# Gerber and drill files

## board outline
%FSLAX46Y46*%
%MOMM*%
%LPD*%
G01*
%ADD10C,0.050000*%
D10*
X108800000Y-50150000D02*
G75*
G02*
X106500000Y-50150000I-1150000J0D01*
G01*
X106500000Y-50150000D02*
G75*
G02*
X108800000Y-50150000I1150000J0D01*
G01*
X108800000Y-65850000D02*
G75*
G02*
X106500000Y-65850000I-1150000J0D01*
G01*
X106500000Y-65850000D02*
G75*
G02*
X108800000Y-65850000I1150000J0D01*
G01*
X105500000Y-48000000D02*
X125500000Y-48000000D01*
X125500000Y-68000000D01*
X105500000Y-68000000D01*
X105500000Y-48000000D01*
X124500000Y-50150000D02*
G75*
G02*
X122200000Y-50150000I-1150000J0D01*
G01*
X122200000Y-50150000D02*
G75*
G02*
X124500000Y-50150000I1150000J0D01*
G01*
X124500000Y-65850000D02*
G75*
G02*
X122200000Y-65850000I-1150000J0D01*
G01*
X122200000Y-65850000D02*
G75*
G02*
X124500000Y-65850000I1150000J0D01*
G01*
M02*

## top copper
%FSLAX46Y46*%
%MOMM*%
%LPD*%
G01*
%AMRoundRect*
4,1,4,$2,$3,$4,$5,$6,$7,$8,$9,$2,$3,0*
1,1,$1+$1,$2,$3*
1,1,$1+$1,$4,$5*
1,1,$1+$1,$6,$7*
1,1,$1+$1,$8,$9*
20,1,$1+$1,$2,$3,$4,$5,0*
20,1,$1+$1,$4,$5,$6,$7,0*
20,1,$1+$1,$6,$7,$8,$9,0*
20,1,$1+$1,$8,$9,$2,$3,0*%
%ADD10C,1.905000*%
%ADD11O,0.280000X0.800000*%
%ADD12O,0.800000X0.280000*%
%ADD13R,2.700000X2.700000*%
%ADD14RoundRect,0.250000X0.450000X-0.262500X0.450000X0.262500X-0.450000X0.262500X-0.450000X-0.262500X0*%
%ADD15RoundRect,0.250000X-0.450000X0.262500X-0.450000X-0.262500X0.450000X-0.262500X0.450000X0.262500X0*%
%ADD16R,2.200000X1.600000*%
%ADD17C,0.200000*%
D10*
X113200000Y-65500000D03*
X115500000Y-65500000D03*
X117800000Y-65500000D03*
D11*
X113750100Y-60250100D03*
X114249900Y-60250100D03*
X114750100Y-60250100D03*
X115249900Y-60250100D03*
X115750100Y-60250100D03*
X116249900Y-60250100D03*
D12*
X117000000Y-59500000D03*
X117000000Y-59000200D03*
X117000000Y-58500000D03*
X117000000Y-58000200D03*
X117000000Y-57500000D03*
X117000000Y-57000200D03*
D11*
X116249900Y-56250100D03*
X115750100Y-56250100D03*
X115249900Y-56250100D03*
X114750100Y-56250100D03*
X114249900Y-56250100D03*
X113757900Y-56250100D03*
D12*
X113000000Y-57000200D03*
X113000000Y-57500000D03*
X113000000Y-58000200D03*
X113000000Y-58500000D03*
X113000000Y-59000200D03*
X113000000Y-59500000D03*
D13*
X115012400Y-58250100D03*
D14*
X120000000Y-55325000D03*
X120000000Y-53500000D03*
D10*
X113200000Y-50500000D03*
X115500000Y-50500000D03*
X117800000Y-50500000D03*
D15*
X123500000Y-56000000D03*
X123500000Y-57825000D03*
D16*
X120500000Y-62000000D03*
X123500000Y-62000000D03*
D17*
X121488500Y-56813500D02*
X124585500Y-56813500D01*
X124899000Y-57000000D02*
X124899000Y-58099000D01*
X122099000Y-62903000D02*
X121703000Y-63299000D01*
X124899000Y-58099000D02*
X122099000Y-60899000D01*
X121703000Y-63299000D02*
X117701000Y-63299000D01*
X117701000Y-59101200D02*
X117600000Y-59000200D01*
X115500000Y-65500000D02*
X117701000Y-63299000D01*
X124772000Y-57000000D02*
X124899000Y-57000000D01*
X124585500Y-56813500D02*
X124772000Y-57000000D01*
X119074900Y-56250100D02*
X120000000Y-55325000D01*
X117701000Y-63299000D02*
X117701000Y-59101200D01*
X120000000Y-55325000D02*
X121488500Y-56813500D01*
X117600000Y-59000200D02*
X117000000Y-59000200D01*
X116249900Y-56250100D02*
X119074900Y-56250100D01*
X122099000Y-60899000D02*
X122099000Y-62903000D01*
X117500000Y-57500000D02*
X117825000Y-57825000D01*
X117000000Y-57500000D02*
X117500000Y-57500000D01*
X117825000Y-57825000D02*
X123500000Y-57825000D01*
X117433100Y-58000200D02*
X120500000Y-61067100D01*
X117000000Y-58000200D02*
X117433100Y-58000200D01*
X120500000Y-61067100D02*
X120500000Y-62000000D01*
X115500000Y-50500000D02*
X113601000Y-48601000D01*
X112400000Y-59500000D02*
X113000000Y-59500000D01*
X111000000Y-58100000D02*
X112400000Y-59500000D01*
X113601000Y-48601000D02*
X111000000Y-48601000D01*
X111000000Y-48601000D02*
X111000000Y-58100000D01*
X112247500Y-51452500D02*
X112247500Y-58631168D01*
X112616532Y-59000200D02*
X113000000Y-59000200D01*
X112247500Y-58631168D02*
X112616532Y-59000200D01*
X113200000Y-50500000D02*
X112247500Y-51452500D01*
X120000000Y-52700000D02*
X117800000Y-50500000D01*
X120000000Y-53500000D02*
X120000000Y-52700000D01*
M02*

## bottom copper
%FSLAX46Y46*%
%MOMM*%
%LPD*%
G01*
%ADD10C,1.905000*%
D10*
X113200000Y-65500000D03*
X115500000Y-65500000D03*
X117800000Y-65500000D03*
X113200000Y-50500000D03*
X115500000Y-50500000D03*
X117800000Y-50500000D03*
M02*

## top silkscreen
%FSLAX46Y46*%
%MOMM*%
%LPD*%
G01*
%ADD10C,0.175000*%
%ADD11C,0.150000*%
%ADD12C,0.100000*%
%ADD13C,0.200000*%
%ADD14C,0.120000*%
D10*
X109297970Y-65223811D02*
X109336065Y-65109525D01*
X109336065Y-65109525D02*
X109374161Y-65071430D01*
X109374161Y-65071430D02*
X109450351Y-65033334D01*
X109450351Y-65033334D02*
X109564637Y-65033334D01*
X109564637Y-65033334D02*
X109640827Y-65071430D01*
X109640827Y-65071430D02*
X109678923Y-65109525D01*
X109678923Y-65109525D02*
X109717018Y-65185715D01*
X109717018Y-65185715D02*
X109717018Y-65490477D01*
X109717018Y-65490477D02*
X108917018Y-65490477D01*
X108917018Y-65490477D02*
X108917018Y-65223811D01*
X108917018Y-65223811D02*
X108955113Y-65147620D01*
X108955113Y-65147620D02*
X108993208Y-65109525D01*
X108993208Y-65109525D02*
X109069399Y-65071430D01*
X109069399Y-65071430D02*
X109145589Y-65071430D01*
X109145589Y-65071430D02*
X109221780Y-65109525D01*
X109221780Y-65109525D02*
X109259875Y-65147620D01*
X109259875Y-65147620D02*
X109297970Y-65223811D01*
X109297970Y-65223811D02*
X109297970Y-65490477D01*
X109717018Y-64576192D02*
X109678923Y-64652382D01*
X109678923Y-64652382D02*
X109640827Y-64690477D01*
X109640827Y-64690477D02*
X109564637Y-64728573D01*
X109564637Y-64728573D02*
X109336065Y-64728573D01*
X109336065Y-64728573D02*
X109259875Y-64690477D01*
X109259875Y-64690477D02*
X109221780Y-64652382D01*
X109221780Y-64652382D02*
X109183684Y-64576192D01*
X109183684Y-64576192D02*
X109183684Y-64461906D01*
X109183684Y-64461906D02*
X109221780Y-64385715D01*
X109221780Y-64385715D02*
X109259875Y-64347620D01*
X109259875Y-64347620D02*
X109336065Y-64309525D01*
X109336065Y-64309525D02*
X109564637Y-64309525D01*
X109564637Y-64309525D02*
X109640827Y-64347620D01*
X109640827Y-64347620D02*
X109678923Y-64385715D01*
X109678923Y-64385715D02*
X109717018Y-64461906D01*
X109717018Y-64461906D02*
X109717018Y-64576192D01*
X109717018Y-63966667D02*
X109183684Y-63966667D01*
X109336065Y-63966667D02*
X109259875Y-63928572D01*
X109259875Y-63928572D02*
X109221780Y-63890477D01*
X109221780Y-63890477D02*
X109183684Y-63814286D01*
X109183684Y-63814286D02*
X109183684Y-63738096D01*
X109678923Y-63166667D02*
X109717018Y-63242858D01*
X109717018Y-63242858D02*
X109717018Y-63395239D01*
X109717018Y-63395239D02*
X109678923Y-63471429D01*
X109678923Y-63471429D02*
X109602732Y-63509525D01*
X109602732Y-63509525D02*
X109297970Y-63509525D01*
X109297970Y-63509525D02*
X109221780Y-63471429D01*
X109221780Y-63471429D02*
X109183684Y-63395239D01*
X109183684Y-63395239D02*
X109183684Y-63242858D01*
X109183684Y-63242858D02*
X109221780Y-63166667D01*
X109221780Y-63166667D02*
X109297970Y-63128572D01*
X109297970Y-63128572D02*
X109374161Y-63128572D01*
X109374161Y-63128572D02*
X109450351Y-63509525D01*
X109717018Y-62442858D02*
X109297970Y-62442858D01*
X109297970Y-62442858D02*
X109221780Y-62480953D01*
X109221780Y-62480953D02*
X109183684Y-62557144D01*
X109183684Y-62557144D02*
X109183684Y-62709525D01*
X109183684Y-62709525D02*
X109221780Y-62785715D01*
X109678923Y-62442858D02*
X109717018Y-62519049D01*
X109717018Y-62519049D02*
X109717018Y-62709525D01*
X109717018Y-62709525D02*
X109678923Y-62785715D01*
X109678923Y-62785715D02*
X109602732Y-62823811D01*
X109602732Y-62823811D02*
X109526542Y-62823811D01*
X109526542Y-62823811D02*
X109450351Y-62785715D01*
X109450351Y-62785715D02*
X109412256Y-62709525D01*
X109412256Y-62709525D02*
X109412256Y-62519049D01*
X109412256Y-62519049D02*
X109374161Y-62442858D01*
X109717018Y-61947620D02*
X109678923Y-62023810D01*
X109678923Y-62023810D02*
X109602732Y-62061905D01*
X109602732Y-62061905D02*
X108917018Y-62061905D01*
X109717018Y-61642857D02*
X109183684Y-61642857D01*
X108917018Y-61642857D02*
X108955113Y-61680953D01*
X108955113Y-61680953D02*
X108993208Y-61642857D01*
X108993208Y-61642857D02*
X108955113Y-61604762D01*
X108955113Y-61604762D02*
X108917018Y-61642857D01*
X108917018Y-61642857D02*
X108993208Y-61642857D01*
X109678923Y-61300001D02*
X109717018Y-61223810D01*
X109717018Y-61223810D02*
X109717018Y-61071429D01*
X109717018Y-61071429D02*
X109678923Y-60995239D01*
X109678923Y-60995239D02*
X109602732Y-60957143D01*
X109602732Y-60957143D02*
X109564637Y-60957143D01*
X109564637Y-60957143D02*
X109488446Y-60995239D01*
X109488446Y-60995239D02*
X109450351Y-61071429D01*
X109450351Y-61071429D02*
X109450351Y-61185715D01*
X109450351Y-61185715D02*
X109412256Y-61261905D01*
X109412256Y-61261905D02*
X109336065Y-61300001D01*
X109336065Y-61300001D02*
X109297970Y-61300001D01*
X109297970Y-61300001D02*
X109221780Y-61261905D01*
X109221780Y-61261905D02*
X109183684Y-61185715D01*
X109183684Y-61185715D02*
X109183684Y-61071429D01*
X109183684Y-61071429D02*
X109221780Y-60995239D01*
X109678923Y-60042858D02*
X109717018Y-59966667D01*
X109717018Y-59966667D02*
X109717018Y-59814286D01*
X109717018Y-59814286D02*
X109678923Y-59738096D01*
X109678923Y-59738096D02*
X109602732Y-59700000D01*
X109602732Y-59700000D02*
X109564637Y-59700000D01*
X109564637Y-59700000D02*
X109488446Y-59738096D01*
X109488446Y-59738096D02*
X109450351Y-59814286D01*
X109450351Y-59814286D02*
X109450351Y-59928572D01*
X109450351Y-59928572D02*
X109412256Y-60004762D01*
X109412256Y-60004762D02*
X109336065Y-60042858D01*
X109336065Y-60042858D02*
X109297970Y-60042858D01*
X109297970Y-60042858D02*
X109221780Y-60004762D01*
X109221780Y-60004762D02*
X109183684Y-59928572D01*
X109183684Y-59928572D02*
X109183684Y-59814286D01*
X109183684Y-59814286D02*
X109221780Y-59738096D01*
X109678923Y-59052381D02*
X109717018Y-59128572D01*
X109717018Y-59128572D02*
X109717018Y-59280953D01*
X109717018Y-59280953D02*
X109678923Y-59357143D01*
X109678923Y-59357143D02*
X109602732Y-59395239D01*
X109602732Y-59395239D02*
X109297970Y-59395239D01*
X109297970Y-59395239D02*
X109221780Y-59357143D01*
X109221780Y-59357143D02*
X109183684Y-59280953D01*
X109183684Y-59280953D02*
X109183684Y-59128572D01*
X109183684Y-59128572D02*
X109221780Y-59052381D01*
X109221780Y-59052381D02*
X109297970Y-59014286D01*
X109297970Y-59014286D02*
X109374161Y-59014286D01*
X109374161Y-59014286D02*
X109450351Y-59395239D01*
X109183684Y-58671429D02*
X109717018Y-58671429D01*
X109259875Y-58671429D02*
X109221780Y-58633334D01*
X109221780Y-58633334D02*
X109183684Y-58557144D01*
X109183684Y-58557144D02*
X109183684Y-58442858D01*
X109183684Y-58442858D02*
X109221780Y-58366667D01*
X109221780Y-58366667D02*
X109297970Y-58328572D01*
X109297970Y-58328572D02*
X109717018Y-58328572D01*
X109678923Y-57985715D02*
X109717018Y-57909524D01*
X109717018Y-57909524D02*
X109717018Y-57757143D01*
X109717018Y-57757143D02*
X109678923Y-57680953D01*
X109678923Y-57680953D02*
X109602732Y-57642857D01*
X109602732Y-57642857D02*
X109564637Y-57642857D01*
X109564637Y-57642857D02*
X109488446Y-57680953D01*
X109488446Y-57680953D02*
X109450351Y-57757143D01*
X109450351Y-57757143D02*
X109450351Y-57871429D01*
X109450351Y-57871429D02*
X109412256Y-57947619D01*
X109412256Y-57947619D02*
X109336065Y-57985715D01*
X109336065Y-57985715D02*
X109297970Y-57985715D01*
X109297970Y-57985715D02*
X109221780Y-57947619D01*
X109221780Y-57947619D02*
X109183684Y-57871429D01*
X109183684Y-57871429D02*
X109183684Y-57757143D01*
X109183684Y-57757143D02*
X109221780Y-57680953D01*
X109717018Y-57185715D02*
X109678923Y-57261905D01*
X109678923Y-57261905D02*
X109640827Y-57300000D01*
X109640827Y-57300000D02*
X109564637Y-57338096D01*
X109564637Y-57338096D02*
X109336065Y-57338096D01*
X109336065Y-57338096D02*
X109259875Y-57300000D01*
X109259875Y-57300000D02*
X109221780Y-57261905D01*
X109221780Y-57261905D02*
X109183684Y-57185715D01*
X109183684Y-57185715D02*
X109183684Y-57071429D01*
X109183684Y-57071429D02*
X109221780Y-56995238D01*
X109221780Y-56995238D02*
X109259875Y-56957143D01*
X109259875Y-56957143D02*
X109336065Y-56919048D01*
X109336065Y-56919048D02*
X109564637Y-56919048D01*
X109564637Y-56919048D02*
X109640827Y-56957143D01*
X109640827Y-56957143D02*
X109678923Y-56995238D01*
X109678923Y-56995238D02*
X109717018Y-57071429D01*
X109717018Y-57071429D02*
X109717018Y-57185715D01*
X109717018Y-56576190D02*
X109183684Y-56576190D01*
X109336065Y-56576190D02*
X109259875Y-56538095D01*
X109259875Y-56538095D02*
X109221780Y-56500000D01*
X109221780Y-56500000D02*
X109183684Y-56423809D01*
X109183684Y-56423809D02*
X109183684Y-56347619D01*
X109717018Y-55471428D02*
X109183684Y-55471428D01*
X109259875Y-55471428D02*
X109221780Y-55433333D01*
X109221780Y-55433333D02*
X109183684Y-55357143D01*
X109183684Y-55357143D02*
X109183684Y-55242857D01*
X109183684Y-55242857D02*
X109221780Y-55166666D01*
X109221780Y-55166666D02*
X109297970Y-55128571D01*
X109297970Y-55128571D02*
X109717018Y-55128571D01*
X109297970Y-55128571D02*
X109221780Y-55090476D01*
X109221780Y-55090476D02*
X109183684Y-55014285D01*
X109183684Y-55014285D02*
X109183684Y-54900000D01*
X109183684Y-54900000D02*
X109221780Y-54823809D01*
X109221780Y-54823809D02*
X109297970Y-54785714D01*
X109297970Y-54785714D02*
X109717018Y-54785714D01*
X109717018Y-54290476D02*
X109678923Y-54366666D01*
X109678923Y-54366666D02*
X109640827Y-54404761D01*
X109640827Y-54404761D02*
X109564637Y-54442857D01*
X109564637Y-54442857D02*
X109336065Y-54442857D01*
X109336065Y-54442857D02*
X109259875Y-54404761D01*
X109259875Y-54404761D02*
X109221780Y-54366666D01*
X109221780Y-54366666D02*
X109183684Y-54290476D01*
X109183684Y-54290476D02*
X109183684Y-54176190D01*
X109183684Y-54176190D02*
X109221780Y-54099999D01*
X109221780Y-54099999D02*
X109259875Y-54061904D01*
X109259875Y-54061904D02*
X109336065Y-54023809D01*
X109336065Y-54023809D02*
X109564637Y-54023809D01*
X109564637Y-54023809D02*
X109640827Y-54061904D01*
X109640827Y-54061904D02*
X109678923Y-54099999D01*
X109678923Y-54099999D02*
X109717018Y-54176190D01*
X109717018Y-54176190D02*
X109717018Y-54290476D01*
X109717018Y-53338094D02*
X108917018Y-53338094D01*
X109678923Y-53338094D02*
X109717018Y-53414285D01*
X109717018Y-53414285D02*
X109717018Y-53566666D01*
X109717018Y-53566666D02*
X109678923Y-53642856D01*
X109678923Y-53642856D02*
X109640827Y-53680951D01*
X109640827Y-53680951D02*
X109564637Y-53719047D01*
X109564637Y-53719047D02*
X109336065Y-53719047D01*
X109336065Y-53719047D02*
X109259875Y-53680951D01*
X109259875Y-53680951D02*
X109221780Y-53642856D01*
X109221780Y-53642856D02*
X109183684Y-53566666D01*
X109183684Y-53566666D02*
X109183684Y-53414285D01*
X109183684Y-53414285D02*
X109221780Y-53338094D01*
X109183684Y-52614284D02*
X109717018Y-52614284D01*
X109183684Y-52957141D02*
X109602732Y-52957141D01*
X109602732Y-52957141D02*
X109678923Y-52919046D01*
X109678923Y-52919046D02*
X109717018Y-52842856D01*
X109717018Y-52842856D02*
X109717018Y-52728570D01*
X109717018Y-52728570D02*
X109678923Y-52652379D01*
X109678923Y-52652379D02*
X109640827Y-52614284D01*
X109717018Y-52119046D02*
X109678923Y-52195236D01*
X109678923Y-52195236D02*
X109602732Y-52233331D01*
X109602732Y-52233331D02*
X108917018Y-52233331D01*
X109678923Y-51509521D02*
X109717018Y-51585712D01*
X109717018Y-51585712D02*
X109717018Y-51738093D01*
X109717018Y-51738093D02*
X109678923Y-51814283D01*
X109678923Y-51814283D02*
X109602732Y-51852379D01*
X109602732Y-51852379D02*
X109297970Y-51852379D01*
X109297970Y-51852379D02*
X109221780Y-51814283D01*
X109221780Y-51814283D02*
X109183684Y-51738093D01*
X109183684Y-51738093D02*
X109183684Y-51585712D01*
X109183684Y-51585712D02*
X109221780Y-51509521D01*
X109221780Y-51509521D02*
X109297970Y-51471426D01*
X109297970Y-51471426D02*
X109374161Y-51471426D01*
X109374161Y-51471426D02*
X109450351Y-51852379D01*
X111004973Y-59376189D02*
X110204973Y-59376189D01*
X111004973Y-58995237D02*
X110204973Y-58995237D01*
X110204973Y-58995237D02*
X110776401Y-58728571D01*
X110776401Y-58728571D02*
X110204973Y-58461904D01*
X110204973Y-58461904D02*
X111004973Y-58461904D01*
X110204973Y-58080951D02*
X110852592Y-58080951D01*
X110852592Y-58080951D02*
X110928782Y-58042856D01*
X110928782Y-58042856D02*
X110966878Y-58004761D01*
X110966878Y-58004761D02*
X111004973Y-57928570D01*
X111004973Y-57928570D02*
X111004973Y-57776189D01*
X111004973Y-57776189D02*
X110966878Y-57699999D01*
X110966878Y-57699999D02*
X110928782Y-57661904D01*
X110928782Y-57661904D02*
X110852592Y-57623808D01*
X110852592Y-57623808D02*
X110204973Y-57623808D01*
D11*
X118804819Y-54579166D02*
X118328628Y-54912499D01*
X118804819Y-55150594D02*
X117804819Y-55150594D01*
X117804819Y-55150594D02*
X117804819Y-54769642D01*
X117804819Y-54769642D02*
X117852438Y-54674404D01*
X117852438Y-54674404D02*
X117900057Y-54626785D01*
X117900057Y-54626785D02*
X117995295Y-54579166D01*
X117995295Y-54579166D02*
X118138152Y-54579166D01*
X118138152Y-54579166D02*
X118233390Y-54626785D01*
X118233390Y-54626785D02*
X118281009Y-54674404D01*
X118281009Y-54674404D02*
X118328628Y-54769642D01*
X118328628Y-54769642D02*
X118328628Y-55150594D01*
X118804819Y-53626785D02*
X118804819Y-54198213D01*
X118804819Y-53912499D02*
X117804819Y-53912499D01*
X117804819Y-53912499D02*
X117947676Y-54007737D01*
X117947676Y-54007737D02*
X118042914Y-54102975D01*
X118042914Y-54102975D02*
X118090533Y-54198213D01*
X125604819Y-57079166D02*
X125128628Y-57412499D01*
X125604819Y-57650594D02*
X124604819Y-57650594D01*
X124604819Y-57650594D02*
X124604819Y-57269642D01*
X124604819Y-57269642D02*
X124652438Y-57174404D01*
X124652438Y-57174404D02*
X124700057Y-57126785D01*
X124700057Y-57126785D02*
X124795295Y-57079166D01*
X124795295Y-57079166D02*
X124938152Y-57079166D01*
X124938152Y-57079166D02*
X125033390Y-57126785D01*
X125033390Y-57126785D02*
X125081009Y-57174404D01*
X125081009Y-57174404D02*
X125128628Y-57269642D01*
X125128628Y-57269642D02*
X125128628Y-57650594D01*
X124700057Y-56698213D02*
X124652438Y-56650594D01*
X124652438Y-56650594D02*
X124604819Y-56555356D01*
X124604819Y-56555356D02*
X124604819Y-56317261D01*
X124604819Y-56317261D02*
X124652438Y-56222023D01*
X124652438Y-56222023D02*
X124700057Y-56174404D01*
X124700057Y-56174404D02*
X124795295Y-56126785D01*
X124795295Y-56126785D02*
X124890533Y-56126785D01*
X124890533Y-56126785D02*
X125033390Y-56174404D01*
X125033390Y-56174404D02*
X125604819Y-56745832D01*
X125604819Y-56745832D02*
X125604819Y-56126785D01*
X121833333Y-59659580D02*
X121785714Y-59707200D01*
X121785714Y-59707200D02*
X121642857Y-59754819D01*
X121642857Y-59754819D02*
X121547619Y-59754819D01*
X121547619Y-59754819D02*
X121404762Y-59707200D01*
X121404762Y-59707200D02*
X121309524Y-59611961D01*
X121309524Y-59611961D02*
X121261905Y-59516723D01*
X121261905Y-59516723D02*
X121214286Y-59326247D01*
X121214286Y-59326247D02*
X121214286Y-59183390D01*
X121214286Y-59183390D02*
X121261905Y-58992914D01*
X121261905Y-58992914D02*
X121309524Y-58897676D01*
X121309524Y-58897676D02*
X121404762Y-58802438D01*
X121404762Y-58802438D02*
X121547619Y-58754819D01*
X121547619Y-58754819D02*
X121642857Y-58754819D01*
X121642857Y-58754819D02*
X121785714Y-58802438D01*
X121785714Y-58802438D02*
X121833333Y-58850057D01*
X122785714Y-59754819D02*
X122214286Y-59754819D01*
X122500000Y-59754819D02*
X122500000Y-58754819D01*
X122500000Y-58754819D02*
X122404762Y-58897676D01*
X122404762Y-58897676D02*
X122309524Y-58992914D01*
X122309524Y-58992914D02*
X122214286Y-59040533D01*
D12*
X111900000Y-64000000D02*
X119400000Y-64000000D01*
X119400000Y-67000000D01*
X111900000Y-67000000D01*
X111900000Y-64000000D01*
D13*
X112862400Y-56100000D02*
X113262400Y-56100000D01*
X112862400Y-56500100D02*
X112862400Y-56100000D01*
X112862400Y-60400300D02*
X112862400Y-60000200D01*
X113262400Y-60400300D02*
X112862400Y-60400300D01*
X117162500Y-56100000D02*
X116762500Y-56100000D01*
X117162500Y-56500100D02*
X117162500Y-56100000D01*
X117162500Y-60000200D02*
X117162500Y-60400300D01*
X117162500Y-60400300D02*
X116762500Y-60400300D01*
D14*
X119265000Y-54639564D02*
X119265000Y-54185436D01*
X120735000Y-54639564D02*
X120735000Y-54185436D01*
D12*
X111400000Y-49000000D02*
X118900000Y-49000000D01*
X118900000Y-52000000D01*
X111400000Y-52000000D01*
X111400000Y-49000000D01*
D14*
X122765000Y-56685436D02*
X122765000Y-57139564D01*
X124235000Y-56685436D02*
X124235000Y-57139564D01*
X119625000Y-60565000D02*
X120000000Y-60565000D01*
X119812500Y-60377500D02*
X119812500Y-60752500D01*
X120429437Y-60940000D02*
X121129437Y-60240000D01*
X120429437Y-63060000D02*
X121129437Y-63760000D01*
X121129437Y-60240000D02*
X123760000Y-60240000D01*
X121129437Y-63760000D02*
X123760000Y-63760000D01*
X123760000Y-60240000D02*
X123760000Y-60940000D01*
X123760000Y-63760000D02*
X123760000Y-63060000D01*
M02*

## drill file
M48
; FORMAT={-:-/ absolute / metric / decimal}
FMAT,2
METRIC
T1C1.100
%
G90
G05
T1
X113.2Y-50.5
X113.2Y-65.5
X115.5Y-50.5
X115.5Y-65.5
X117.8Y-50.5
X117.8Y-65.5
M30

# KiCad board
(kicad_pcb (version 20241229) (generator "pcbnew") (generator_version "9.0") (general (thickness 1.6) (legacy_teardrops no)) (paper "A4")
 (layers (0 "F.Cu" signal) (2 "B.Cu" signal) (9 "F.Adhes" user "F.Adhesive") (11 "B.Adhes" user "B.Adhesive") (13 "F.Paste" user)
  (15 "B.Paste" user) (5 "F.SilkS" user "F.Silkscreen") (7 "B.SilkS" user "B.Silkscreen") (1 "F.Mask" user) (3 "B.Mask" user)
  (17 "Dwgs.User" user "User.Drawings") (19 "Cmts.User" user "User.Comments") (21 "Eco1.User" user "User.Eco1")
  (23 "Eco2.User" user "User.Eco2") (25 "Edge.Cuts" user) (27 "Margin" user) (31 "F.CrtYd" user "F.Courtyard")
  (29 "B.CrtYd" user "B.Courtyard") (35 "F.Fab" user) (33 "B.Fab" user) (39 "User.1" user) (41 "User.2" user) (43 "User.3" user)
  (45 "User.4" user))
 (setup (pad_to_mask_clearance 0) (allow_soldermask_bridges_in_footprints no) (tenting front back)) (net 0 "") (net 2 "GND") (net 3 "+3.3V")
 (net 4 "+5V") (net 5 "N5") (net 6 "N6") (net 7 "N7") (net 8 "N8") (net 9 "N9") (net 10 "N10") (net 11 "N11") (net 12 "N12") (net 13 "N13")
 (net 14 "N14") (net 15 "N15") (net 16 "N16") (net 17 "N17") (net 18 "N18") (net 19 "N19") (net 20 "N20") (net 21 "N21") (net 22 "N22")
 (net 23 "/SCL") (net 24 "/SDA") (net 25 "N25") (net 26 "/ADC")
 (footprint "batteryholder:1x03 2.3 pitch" (layer "F.Cu") (at 113.4 65.5)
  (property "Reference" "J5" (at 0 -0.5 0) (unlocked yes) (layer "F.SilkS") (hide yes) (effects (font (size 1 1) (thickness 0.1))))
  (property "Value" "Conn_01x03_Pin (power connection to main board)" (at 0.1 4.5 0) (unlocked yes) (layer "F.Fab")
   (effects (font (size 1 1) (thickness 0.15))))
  (fp_rect (start -1.5 -1.5) (end 6 1.5) (stroke (width 0.1) (type default)) (fill no) (layer "F.SilkS") (net 1))
  (pad "1" thru_hole circle (at -0.2 0) (size 1.905 1.905) (drill 1.1) (layers "*.Cu" "*.Mask") (remove_unused_layers no) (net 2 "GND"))
  (pad "2" thru_hole circle (at 2.1 0) (size 1.905 1.905) (drill 1.1) (layers "*.Cu" "*.Mask") (remove_unused_layers no) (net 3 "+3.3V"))
  (pad "3" thru_hole circle (at 4.4 0) (size 1.905 1.905) (drill 1.1) (layers "*.Cu" "*.Mask") (remove_unused_layers no) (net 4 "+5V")))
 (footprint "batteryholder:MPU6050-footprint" (layer "F.Cu") (at 115 58.2501)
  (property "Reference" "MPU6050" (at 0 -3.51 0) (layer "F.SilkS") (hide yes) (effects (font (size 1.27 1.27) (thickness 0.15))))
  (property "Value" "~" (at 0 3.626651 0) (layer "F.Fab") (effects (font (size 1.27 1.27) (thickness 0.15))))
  (fp_line (start -2.1376 -2.1501) (end -1.7376 -2.1501) (stroke (width 0.2) (type default)) (layer "F.SilkS"))
  (fp_line (start -2.1376 -1.75) (end -2.1376 -2.1501) (stroke (width 0.2) (type default)) (layer "F.SilkS"))
  (fp_line (start -2.1376 2.1502) (end -2.1376 1.7501) (stroke (width 0.2) (type default)) (layer "F.SilkS"))
  (fp_line (start -1.7376 2.1502) (end -2.1376 2.1502) (stroke (width 0.2) (type default)) (layer "F.SilkS"))
  (fp_line (start 2.1625 -2.1501) (end 1.7625 -2.1501) (stroke (width 0.2) (type default)) (layer "F.SilkS"))
  (fp_line (start 2.1625 -1.75) (end 2.1625 -2.1501) (stroke (width 0.2) (type default)) (layer "F.SilkS"))
  (fp_line (start 2.1625 1.7501) (end 2.1625 2.1502) (stroke (width 0.2) (type default)) (layer "F.SilkS"))
  (fp_line (start 2.1625 2.1502) (end 1.7625 2.1502) (stroke (width 0.2) (type default)) (layer "F.SilkS"))
  (pad "1" smd oval (at -1.2499 2) (size 0.28 0.8) (layers "F.Cu" "F.Mask" "F.Paste") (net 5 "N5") (solder_mask_margin 0.05)
   (solder_paste_margin -99.9998) (thermal_bridge_angle 0))
  (pad "2" smd oval (at -0.7501 2) (size 0.28 0.8) (layers "F.Cu" "F.Mask" "F.Paste") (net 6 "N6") (solder_mask_margin 0.05)
   (solder_paste_margin -99.9998) (thermal_bridge_angle 0))
  (pad "3" smd oval (at -0.2499 2) (size 0.28 0.8) (layers "F.Cu" "F.Mask" "F.Paste") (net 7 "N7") (solder_mask_margin 0.05)
   (solder_paste_margin -99.9998) (thermal_bridge_angle 0))
  (pad "4" smd oval (at 0.2499 2) (size 0.28 0.8) (layers "F.Cu" "F.Mask" "F.Paste") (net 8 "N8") (solder_mask_margin 0.05)
   (solder_paste_margin -99.9998) (thermal_bridge_angle 0))
  (pad "5" smd oval (at 0.7501 2) (size 0.28 0.8) (layers "F.Cu" "F.Mask" "F.Paste") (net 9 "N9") (solder_mask_margin 0.05)
   (solder_paste_margin -99.9998) (thermal_bridge_angle 0))
  (pad "6" smd oval (at 1.2499 2) (size 0.28 0.8) (layers "F.Cu" "F.Mask" "F.Paste") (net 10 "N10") (solder_mask_margin 0.05)
   (solder_paste_margin -99.9998) (thermal_bridge_angle 0))
  (pad "7" smd oval (at 2 1.2499) (size 0.8 0.28) (layers "F.Cu" "F.Mask" "F.Paste") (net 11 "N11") (solder_mask_margin 0.05)
   (solder_paste_margin -99.9998) (thermal_bridge_angle 0))
  (pad "8" smd oval (at 2 0.7501) (size 0.8 0.28) (layers "F.Cu" "F.Mask" "F.Paste") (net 3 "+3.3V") (solder_mask_margin 0.05)
   (solder_paste_margin -99.9998) (thermal_bridge_angle 0))
  (pad "9" smd oval (at 2 0.2499) (size 0.8 0.28) (layers "F.Cu" "F.Mask" "F.Paste") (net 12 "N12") (solder_mask_margin 0.05)
   (solder_paste_margin -99.9998) (thermal_bridge_angle 0))
  (pad "10" smd oval (at 2 -0.2499) (size 0.8 0.28) (layers "F.Cu" "F.Mask" "F.Paste") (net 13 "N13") (solder_mask_margin 0.05)
   (solder_paste_margin -99.9998) (thermal_bridge_angle 0))
  (pad "11" smd oval (at 2 -0.7501) (size 0.8 0.28) (layers "F.Cu" "F.Mask" "F.Paste") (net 12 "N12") (solder_mask_margin 0.05)
   (solder_paste_margin -99.9998) (thermal_bridge_angle 0))
  (pad "12" smd oval (at 2 -1.2499) (size 0.8 0.28) (layers "F.Cu" "F.Mask" "F.Paste") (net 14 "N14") (solder_mask_margin 0.05)
   (solder_paste_margin -99.9998) (thermal_bridge_angle 0))
  (pad "13" smd oval (at 1.2499 -2) (size 0.28 0.8) (layers "F.Cu" "F.Mask" "F.Paste") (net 3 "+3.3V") (solder_mask_margin 0.05)
   (solder_paste_margin -99.9998) (thermal_bridge_angle 0))
  (pad "14" smd oval (at 0.7501 -2) (size 0.28 0.8) (layers "F.Cu" "F.Mask" "F.Paste") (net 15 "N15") (solder_mask_margin 0.05)
   (solder_paste_margin -99.9998) (thermal_bridge_angle 0))
  (pad "15" smd oval (at 0.2499 -2) (size 0.28 0.8) (layers "F.Cu" "F.Mask" "F.Paste") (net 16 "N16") (solder_mask_margin 0.05)
   (solder_paste_margin -99.9998) (thermal_bridge_angle 0))
  (pad "16" smd oval (at -0.2499 -2) (size 0.28 0.8) (layers "F.Cu" "F.Mask" "F.Paste") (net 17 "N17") (solder_mask_margin 0.05)
   (solder_paste_margin -99.9998) (thermal_bridge_angle 0))
  (pad "17" smd oval (at -0.7501 -2) (size 0.28 0.8) (layers "F.Cu" "F.Mask" "F.Paste") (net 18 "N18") (solder_mask_margin 0.05)
   (solder_paste_margin -99.9998) (thermal_bridge_angle 0))
  (pad "18" smd oval (at -1.2421 -2) (size 0.28 0.8) (layers "F.Cu" "F.Mask" "F.Paste") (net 2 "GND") (solder_mask_margin 0.05)
   (solder_paste_margin -99.9998) (thermal_bridge_angle 0))
  (pad "19" smd oval (at -2 -1.2499) (size 0.8 0.28) (layers "F.Cu" "F.Mask" "F.Paste") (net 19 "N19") (solder_mask_margin 0.05)
   (solder_paste_margin -99.9998) (thermal_bridge_angle 0))
  (pad "20" smd oval (at -2 -0.7501) (size 0.8 0.28) (layers "F.Cu" "F.Mask" "F.Paste") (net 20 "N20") (solder_mask_margin 0.05)
   (solder_paste_margin -99.9998) (thermal_bridge_angle 0))
  (pad "21" smd oval (at -2 -0.2499) (size 0.8 0.28) (layers "F.Cu" "F.Mask" "F.Paste") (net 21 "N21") (solder_mask_margin 0.05)
   (solder_paste_margin -99.9998) (thermal_bridge_angle 0))
  (pad "22" smd oval (at -2 0.2499) (size 0.8 0.28) (layers "F.Cu" "F.Mask" "F.Paste") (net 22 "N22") (solder_mask_margin 0.05)
   (solder_paste_margin -99.9998) (thermal_bridge_angle 0))
  (pad "23" smd oval (at -2 0.7501) (size 0.8 0.28) (layers "F.Cu" "F.Mask" "F.Paste") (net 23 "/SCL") (solder_mask_margin 0.05)
   (solder_paste_margin -99.9998) (thermal_bridge_angle 0))
  (pad "24" smd oval (at -2 1.2499) (size 0.8 0.28) (layers "F.Cu" "F.Mask" "F.Paste") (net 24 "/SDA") (solder_mask_margin 0.05)
   (solder_paste_margin -99.9998) (thermal_bridge_angle 0))
  (pad "25" smd rect (at 0.0124 0) (size 2.7 2.7) (layers "F.Cu" "F.Mask" "F.Paste") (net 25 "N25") (solder_mask_margin 0.05)
   (solder_paste_margin -99.9998) (thermal_bridge_angle 0))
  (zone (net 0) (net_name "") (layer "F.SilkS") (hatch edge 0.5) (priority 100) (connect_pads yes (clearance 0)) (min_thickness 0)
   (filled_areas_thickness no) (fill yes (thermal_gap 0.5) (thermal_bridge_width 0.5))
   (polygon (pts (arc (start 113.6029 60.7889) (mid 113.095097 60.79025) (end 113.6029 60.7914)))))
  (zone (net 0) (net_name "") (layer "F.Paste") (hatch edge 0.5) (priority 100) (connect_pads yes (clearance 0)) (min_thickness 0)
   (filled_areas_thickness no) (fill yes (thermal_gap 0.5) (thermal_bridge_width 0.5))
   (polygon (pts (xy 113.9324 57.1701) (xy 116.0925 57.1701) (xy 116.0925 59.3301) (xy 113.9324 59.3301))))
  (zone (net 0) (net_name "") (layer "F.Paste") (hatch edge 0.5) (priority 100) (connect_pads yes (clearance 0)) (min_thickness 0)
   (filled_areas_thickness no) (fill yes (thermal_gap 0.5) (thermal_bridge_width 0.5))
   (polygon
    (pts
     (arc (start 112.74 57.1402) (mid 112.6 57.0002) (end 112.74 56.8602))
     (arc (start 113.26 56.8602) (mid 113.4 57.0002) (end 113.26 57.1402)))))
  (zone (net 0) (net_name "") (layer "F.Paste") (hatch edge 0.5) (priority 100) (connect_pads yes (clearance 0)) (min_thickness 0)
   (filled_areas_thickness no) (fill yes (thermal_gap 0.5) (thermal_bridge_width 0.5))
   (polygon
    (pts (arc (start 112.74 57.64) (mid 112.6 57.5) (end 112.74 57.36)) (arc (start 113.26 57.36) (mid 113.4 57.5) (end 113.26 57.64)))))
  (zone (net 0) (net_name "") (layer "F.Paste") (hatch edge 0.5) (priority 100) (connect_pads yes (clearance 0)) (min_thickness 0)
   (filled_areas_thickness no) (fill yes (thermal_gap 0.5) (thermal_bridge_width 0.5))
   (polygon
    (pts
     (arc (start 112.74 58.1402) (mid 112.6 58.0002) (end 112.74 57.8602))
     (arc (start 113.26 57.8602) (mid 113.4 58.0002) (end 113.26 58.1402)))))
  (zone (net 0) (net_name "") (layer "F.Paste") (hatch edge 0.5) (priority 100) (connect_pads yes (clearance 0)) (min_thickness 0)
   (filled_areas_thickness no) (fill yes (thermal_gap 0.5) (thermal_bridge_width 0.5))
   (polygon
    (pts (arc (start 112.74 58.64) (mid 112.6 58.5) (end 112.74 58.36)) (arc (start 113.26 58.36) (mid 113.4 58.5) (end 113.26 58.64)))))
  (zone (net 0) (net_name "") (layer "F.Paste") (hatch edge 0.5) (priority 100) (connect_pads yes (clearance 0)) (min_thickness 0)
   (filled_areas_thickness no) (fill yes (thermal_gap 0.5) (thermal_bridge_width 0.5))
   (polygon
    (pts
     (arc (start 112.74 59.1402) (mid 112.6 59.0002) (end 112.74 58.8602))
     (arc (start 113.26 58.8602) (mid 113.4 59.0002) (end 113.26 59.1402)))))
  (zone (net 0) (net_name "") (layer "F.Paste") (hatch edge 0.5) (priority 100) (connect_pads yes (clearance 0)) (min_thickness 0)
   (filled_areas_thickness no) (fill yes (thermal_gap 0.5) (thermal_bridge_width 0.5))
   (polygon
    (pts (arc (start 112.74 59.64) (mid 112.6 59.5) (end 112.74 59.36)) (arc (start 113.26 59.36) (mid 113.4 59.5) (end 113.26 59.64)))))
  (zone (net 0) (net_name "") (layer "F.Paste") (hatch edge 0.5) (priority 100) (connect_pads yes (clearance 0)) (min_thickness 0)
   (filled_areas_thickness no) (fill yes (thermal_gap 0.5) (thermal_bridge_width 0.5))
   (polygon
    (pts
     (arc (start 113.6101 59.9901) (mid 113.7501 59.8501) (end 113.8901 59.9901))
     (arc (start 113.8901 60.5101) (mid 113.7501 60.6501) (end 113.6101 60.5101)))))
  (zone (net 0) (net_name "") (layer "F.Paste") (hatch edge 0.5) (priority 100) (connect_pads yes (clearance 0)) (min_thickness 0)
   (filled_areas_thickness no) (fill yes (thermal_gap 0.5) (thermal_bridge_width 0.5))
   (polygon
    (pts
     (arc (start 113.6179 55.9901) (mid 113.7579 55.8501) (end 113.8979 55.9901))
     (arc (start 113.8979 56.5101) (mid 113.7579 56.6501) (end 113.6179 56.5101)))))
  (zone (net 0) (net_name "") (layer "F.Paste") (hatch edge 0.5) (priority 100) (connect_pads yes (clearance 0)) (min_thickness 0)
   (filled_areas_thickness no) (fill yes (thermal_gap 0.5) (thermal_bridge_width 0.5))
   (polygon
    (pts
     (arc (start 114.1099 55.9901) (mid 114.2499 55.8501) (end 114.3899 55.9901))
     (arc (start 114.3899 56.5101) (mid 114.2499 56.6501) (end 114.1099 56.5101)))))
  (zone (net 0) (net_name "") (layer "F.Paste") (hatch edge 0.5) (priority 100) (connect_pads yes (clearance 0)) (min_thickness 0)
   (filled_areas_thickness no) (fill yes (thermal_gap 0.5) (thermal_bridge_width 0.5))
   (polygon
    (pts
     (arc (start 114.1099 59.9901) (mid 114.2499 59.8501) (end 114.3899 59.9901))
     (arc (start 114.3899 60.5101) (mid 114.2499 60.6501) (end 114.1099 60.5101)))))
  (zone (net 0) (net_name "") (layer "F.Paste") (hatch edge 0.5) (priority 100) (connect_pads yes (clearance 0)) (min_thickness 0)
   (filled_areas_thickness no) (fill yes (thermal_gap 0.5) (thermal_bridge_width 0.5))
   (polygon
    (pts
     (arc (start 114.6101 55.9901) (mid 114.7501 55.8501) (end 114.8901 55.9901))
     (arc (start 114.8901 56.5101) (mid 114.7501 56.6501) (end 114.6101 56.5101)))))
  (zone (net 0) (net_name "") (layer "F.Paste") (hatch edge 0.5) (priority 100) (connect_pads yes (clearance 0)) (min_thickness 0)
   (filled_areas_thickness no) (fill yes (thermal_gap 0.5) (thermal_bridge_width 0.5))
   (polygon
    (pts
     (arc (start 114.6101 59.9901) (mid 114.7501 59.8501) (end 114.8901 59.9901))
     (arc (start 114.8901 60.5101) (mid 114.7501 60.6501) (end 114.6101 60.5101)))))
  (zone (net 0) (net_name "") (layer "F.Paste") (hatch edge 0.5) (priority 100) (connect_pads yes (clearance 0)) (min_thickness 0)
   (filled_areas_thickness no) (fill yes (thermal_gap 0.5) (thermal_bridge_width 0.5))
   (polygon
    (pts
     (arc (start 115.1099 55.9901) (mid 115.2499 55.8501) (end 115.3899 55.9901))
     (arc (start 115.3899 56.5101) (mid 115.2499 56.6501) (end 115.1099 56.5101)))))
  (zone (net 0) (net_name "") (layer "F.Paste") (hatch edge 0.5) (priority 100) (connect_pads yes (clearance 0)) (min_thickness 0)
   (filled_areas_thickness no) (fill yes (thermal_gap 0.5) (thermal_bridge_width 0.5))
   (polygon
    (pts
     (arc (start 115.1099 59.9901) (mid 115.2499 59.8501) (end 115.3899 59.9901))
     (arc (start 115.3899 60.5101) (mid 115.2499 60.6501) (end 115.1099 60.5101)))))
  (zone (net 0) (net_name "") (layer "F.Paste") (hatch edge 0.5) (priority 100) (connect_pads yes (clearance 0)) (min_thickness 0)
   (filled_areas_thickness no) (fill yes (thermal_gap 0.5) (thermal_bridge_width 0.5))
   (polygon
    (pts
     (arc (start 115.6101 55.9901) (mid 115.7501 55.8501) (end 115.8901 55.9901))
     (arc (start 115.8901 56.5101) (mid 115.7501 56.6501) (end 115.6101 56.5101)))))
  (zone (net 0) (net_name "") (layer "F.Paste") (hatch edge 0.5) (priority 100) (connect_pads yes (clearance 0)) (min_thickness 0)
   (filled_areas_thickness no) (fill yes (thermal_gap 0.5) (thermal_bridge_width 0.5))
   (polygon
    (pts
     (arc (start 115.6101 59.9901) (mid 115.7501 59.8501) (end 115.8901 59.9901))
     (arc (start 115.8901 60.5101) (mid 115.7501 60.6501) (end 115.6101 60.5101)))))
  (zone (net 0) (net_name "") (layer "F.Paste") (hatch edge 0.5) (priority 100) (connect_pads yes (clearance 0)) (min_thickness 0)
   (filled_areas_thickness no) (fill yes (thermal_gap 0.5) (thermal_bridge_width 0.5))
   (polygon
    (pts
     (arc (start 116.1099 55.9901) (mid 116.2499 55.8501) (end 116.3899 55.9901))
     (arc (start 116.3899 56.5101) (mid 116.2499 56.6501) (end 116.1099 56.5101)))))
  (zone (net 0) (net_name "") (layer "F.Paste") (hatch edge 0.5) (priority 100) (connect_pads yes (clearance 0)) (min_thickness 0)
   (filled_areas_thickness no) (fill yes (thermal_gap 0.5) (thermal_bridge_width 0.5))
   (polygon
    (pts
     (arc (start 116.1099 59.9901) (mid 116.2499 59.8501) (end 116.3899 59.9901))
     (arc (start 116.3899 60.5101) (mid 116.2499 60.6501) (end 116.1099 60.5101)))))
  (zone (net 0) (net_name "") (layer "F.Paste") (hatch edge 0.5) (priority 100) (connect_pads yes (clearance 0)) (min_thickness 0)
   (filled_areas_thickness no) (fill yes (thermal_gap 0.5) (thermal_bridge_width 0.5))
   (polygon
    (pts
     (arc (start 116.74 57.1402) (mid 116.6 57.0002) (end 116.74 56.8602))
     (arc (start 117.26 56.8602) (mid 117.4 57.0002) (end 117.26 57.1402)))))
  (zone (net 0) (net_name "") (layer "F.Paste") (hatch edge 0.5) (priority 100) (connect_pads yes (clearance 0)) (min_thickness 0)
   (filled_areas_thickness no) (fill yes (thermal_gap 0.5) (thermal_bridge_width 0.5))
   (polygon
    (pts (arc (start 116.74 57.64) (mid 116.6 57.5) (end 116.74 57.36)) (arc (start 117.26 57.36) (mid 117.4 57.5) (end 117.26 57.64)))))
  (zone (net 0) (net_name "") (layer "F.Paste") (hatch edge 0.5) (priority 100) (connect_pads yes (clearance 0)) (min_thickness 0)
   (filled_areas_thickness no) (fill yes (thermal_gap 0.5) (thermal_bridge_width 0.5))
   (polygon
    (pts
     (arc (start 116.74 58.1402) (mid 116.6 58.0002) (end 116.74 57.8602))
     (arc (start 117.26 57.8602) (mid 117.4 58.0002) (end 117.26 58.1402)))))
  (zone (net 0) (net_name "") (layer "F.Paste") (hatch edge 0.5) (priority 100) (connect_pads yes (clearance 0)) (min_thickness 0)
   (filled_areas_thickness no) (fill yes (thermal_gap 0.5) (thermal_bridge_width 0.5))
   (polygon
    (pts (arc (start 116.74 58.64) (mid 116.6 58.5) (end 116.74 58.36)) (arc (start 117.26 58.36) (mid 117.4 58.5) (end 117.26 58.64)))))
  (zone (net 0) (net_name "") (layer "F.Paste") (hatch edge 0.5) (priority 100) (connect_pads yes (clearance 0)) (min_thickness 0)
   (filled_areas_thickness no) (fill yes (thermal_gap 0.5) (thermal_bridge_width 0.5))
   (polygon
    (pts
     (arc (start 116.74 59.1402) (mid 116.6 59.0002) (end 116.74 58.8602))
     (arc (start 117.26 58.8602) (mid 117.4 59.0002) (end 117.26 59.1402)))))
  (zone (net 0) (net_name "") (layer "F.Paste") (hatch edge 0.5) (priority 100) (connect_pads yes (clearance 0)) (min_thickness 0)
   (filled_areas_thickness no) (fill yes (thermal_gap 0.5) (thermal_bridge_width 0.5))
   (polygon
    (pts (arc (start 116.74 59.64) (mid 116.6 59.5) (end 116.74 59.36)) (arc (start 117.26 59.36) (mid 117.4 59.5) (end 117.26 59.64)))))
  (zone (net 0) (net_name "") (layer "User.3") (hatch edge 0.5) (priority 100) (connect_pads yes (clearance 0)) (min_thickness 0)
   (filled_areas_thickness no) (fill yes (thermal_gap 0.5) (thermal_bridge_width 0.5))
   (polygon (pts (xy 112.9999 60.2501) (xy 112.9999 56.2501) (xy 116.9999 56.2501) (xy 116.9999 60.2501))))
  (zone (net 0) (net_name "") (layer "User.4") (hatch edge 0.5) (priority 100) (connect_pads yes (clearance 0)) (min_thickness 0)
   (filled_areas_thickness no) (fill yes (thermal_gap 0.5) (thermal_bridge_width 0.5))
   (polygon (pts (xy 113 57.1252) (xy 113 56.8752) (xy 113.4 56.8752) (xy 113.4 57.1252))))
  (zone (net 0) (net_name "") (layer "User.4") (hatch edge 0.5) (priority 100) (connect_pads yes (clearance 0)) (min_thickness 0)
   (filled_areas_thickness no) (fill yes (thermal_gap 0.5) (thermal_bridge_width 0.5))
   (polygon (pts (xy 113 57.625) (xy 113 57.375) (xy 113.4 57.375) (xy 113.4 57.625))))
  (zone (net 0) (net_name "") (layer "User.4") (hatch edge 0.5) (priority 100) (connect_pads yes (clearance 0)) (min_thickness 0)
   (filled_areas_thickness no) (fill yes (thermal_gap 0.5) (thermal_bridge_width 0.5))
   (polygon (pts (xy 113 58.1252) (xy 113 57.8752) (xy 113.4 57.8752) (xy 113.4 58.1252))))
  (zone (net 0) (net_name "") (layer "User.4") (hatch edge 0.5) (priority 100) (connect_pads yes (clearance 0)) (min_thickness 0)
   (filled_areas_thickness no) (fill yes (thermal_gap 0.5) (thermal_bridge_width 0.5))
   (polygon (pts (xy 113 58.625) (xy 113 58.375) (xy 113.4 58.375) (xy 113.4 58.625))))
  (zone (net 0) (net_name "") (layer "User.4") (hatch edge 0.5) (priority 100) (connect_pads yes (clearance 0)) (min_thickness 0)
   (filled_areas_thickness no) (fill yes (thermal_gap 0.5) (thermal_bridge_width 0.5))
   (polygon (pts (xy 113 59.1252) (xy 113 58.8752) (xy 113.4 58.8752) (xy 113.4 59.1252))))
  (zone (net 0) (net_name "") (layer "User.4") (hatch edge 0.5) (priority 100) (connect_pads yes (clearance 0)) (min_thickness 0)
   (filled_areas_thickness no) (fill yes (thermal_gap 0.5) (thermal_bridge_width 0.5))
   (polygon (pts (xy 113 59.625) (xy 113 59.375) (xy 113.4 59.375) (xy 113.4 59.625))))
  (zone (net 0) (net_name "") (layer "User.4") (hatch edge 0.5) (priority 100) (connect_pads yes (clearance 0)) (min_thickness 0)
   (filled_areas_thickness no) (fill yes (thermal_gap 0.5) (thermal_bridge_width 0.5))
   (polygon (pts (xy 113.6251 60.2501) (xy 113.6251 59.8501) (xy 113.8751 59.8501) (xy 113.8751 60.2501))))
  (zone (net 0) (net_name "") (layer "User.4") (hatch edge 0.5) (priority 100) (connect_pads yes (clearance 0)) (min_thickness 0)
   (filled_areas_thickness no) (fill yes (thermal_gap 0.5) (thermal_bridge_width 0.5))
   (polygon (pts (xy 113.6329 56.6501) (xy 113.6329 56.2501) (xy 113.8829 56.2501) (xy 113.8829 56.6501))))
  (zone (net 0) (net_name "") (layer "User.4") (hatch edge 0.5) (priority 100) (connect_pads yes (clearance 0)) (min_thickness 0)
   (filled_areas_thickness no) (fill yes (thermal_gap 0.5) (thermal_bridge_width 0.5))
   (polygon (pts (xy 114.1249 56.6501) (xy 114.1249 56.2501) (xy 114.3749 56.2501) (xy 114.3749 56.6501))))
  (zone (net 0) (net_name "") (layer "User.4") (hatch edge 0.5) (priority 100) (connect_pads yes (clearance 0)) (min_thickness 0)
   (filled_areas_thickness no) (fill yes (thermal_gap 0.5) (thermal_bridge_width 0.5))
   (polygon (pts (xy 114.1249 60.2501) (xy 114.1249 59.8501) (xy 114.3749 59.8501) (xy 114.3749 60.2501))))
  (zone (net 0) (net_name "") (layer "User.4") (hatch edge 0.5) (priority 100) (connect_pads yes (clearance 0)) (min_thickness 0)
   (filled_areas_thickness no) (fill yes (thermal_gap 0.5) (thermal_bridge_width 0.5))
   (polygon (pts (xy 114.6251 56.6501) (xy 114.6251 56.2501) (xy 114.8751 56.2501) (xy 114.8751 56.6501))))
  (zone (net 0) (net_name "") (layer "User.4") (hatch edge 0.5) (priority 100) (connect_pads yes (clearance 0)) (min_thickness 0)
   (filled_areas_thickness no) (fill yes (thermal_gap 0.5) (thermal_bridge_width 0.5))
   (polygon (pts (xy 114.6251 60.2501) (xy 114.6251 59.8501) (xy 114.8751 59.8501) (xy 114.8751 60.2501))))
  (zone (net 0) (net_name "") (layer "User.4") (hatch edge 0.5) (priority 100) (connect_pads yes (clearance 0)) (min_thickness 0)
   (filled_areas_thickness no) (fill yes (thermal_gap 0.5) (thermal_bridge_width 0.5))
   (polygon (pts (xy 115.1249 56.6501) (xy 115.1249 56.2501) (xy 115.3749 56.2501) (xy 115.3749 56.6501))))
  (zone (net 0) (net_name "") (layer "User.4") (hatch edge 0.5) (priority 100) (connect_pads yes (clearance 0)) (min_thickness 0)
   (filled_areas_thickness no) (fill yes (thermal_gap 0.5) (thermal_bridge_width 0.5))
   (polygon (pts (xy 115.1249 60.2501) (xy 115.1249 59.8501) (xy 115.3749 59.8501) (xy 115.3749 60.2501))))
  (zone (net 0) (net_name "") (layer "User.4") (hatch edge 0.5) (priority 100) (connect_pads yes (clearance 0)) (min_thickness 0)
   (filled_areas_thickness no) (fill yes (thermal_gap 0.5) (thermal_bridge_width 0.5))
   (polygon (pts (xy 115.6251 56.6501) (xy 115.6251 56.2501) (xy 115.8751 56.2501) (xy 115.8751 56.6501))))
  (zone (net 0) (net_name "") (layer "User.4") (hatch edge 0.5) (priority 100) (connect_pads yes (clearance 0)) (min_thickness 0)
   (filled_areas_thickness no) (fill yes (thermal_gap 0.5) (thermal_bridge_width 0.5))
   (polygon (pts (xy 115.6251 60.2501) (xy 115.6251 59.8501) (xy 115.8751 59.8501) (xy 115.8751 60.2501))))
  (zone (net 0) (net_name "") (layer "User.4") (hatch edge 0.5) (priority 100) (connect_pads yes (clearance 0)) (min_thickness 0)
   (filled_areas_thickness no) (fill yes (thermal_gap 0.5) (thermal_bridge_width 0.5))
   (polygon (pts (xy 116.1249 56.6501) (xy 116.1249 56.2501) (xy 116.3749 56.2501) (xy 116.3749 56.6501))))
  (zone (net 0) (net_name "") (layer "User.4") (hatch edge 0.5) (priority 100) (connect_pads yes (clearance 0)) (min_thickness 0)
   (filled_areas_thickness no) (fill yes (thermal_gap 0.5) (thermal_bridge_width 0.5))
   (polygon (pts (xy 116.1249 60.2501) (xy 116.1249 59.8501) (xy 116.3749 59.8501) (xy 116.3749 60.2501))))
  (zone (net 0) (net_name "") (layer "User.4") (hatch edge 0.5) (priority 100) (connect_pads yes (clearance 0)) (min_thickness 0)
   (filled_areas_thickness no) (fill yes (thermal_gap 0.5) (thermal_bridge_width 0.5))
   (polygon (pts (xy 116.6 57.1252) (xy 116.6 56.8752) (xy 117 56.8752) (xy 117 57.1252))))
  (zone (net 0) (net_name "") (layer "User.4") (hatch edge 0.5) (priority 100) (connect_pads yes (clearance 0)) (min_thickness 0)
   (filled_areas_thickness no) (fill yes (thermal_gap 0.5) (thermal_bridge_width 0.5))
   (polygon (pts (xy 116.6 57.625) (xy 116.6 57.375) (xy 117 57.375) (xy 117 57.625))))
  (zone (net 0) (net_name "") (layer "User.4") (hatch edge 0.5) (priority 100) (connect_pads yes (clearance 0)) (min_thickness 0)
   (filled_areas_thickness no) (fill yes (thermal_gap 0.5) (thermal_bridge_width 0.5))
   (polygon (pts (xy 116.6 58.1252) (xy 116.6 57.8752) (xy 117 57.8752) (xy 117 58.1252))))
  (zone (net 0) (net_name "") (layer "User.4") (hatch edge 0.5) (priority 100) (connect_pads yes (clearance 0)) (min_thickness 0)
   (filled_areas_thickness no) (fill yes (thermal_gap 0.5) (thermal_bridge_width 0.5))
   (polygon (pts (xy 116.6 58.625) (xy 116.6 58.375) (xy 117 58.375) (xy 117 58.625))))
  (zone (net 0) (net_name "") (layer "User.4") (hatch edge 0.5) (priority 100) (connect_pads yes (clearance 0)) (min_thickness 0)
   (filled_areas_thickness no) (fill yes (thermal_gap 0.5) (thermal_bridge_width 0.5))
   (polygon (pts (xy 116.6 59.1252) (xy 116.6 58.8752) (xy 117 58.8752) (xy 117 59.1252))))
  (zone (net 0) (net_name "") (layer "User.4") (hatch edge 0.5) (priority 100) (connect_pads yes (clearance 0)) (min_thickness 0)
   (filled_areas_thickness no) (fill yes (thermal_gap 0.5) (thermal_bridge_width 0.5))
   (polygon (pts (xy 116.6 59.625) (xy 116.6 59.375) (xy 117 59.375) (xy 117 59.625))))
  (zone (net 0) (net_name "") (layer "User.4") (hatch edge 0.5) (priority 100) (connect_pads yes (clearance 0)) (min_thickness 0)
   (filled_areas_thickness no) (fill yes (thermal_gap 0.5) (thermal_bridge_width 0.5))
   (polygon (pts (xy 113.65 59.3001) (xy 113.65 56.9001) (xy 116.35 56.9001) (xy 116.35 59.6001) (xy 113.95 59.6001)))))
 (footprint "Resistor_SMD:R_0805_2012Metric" (layer "F.Cu") (at 120 54.4125 90)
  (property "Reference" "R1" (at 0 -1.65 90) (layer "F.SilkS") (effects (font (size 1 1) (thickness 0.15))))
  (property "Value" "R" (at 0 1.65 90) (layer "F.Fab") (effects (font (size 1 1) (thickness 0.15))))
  (fp_line (start -0.227064 -0.735) (end 0.227064 -0.735) (stroke (width 0.12) (type solid)) (layer "F.SilkS"))
  (fp_line (start -0.227064 0.735) (end 0.227064 0.735) (stroke (width 0.12) (type solid)) (layer "F.SilkS"))
  (pad "1" smd roundrect (at -0.9125 0 90) (size 1.025 1.4) (layers "F.Cu" "F.Mask" "F.Paste") (roundrect_rratio 0.243902) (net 3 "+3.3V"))
  (pad "2" smd roundrect (at 0.9125 0 90) (size 1.025 1.4) (layers "F.Cu" "F.Mask" "F.Paste") (roundrect_rratio 0.243902) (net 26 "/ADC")))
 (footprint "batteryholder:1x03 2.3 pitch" (layer "F.Cu") (at 112.9 50.5)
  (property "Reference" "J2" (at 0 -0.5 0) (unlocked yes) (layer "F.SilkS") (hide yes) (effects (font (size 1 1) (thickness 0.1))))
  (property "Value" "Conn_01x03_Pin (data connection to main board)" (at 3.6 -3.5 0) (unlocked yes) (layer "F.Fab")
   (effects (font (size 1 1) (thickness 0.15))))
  (fp_rect (start -1.5 -1.5) (end 6 1.5) (stroke (width 0.1) (type default)) (fill no) (layer "F.SilkS") (net 1))
  (pad "1" thru_hole circle (at 0.3 0) (size 1.905 1.905) (drill 1.1) (layers "*.Cu" "*.Mask") (remove_unused_layers no) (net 23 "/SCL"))
  (pad "2" thru_hole circle (at 2.6 0) (size 1.905 1.905) (drill 1.1) (layers "*.Cu" "*.Mask") (remove_unused_layers no) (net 24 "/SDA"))
  (pad "3" thru_hole circle (at 4.9 0) (size 1.905 1.905) (drill 1.1) (layers "*.Cu" "*.Mask") (remove_unused_layers no) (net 26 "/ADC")))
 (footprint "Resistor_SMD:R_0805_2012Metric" (layer "F.Cu") (at 123.5 56.9125 -90)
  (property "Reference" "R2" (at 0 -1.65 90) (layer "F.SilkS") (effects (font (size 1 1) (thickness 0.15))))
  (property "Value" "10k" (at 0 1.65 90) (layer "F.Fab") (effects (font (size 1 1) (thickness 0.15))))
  (fp_line (start -0.227064 0.735) (end 0.227064 0.735) (stroke (width 0.12) (type solid)) (layer "F.SilkS"))
  (fp_line (start -0.227064 -0.735) (end 0.227064 -0.735) (stroke (width 0.12) (type solid)) (layer "F.SilkS"))
  (pad "1" smd roundrect (at -0.9125 0 270) (size 1.025 1.4) (layers "F.Cu" "F.Mask" "F.Paste") (roundrect_rratio 0.243902) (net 2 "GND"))
  (pad "2" smd roundrect (at 0.9125 0 270) (size 1.025 1.4) (layers "F.Cu" "F.Mask" "F.Paste") (roundrect_rratio 0.243902) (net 12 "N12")))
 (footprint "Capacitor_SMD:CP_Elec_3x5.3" (layer "F.Cu") (at 122 62)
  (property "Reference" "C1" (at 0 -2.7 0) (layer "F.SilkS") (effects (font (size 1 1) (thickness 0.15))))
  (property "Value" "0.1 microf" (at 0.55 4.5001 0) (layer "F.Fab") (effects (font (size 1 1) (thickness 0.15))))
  (fp_line (start -2.375 -1.435) (end -2 -1.435) (stroke (width 0.12) (type solid)) (layer "F.SilkS"))
  (fp_line (start -2.1875 -1.6225) (end -2.1875 -1.2475) (stroke (width 0.12) (type solid)) (layer "F.SilkS"))
  (fp_line (start -1.570563 -1.06) (end -0.870563 -1.76) (stroke (width 0.12) (type solid)) (layer "F.SilkS"))
  (fp_line (start -1.570563 1.06) (end -0.870563 1.76) (stroke (width 0.12) (type solid)) (layer "F.SilkS"))
  (fp_line (start -0.870563 -1.76) (end 1.76 -1.76) (stroke (width 0.12) (type solid)) (layer "F.SilkS"))
  (fp_line (start -0.870563 1.76) (end 1.76 1.76) (stroke (width 0.12) (type solid)) (layer "F.SilkS"))
  (fp_line (start 1.76 -1.76) (end 1.76 -1.06) (stroke (width 0.12) (type solid)) (layer "F.SilkS"))
  (fp_line (start 1.76 1.76) (end 1.76 1.06) (stroke (width 0.12) (type solid)) (layer "F.SilkS"))
  (pad "1" smd rect (at -1.5 0) (size 2.2 1.6) (layers "F.Cu" "F.Mask" "F.Paste") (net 13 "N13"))
  (pad "2" smd rect (at 1.5 0) (size 2.2 1.6) (layers "F.Cu" "F.Mask" "F.Paste") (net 2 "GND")))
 (gr_circle (center 107.65 50.15) (end 108.8 50.15) (stroke (width 0.05) (type solid)) (fill no) (layer "Edge.Cuts"))
 (gr_circle (center 107.65 65.85) (end 108.8 65.85) (stroke (width 0.05) (type solid)) (fill no) (layer "Edge.Cuts"))
 (gr_rect (start 105.5 48) (end 125.5 68) (stroke (width 0.05) (type solid)) (fill no) (layer "Edge.Cuts"))
 (gr_circle (center 123.35 50.15) (end 124.5 50.15) (stroke (width 0.05) (type solid)) (fill no) (layer "Edge.Cuts"))
 (gr_circle (center 123.35 65.85) (end 124.5 65.85) (stroke (width 0.05) (type solid)) (fill no) (layer "Edge.Cuts"))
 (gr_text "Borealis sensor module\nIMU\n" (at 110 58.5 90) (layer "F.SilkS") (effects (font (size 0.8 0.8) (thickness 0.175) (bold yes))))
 (segment (start 121.4885 56.8135) (end 124.5855 56.8135) (width 0.2) (layer "F.Cu") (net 3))
 (segment (start 124.899 57) (end 124.899 58.099) (width 0.2) (layer "F.Cu") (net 3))
 (segment (start 122.099 62.903) (end 121.703 63.299) (width 0.2) (layer "F.Cu") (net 3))
 (segment (start 124.899 58.099) (end 122.099 60.899) (width 0.2) (layer "F.Cu") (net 3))
 (segment (start 121.703 63.299) (end 117.701 63.299) (width 0.2) (layer "F.Cu") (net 3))
 (segment (start 117.701 59.1012) (end 117.6 59.0002) (width 0.2) (layer "F.Cu") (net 3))
 (segment (start 115.5 65.5) (end 117.701 63.299) (width 0.2) (layer "F.Cu") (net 3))
 (segment (start 124.772 57) (end 124.899 57) (width 0.2) (layer "F.Cu") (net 3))
 (segment (start 124.5855 56.8135) (end 124.772 57) (width 0.2) (layer "F.Cu") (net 3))
 (segment (start 119.0749 56.2501) (end 120 55.325) (width 0.2) (layer "F.Cu") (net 3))
 (segment (start 117.701 63.299) (end 117.701 59.1012) (width 0.2) (layer "F.Cu") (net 3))
 (segment (start 120 55.325) (end 121.4885 56.8135) (width 0.2) (layer "F.Cu") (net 3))
 (segment (start 117.6 59.0002) (end 117 59.0002) (width 0.2) (layer "F.Cu") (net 3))
 (segment (start 116.2499 56.2501) (end 119.0749 56.2501) (width 0.2) (layer "F.Cu") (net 3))
 (segment (start 122.099 60.899) (end 122.099 62.903) (width 0.2) (layer "F.Cu") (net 3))
 (segment (start 117.5 57.5) (end 117.825 57.825) (width 0.2) (layer "F.Cu") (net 12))
 (segment (start 117 57.5) (end 117.5 57.5) (width 0.2) (layer "F.Cu") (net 12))
 (segment (start 117.825 57.825) (end 123.5 57.825) (width 0.2) (layer "F.Cu") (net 12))
 (segment (start 117.4331 58.0002) (end 120.5 61.0671) (width 0.2) (layer "F.Cu") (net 13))
 (segment (start 117 58.0002) (end 117.4331 58.0002) (width 0.2) (layer "F.Cu") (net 13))
 (segment (start 120.5 61.0671) (end 120.5 62) (width 0.2) (layer "F.Cu") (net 13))
 (segment (start 115.5 50.5) (end 113.601 48.601) (width 0.2) (layer "F.Cu") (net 24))
 (segment (start 112.4 59.5) (end 113 59.5) (width 0.2) (layer "F.Cu") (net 24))
 (segment (start 111 58.1) (end 112.4 59.5) (width 0.2) (layer "F.Cu") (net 24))
 (segment (start 113.601 48.601) (end 111 48.601) (width 0.2) (layer "F.Cu") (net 24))
 (segment (start 111 48.601) (end 111 58.1) (width 0.2) (layer "F.Cu") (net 24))
 (segment (start 112.2475 51.4525) (end 112.2475 58.631168) (width 0.2) (layer "F.Cu") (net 23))
 (segment (start 112.616532 59.0002) (end 113 59.0002) (width 0.2) (layer "F.Cu") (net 23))
 (segment (start 112.2475 58.631168) (end 112.616532 59.0002) (width 0.2) (layer "F.Cu") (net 23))
 (segment (start 113.2 50.5) (end 112.2475 51.4525) (width 0.2) (layer "F.Cu") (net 23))
 (segment (start 120 52.7) (end 117.8 50.5) (width 0.2) (layer "F.Cu") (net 26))
 (segment (start 120 53.5) (end 120 52.7) (width 0.2) (layer "F.Cu") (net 26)))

